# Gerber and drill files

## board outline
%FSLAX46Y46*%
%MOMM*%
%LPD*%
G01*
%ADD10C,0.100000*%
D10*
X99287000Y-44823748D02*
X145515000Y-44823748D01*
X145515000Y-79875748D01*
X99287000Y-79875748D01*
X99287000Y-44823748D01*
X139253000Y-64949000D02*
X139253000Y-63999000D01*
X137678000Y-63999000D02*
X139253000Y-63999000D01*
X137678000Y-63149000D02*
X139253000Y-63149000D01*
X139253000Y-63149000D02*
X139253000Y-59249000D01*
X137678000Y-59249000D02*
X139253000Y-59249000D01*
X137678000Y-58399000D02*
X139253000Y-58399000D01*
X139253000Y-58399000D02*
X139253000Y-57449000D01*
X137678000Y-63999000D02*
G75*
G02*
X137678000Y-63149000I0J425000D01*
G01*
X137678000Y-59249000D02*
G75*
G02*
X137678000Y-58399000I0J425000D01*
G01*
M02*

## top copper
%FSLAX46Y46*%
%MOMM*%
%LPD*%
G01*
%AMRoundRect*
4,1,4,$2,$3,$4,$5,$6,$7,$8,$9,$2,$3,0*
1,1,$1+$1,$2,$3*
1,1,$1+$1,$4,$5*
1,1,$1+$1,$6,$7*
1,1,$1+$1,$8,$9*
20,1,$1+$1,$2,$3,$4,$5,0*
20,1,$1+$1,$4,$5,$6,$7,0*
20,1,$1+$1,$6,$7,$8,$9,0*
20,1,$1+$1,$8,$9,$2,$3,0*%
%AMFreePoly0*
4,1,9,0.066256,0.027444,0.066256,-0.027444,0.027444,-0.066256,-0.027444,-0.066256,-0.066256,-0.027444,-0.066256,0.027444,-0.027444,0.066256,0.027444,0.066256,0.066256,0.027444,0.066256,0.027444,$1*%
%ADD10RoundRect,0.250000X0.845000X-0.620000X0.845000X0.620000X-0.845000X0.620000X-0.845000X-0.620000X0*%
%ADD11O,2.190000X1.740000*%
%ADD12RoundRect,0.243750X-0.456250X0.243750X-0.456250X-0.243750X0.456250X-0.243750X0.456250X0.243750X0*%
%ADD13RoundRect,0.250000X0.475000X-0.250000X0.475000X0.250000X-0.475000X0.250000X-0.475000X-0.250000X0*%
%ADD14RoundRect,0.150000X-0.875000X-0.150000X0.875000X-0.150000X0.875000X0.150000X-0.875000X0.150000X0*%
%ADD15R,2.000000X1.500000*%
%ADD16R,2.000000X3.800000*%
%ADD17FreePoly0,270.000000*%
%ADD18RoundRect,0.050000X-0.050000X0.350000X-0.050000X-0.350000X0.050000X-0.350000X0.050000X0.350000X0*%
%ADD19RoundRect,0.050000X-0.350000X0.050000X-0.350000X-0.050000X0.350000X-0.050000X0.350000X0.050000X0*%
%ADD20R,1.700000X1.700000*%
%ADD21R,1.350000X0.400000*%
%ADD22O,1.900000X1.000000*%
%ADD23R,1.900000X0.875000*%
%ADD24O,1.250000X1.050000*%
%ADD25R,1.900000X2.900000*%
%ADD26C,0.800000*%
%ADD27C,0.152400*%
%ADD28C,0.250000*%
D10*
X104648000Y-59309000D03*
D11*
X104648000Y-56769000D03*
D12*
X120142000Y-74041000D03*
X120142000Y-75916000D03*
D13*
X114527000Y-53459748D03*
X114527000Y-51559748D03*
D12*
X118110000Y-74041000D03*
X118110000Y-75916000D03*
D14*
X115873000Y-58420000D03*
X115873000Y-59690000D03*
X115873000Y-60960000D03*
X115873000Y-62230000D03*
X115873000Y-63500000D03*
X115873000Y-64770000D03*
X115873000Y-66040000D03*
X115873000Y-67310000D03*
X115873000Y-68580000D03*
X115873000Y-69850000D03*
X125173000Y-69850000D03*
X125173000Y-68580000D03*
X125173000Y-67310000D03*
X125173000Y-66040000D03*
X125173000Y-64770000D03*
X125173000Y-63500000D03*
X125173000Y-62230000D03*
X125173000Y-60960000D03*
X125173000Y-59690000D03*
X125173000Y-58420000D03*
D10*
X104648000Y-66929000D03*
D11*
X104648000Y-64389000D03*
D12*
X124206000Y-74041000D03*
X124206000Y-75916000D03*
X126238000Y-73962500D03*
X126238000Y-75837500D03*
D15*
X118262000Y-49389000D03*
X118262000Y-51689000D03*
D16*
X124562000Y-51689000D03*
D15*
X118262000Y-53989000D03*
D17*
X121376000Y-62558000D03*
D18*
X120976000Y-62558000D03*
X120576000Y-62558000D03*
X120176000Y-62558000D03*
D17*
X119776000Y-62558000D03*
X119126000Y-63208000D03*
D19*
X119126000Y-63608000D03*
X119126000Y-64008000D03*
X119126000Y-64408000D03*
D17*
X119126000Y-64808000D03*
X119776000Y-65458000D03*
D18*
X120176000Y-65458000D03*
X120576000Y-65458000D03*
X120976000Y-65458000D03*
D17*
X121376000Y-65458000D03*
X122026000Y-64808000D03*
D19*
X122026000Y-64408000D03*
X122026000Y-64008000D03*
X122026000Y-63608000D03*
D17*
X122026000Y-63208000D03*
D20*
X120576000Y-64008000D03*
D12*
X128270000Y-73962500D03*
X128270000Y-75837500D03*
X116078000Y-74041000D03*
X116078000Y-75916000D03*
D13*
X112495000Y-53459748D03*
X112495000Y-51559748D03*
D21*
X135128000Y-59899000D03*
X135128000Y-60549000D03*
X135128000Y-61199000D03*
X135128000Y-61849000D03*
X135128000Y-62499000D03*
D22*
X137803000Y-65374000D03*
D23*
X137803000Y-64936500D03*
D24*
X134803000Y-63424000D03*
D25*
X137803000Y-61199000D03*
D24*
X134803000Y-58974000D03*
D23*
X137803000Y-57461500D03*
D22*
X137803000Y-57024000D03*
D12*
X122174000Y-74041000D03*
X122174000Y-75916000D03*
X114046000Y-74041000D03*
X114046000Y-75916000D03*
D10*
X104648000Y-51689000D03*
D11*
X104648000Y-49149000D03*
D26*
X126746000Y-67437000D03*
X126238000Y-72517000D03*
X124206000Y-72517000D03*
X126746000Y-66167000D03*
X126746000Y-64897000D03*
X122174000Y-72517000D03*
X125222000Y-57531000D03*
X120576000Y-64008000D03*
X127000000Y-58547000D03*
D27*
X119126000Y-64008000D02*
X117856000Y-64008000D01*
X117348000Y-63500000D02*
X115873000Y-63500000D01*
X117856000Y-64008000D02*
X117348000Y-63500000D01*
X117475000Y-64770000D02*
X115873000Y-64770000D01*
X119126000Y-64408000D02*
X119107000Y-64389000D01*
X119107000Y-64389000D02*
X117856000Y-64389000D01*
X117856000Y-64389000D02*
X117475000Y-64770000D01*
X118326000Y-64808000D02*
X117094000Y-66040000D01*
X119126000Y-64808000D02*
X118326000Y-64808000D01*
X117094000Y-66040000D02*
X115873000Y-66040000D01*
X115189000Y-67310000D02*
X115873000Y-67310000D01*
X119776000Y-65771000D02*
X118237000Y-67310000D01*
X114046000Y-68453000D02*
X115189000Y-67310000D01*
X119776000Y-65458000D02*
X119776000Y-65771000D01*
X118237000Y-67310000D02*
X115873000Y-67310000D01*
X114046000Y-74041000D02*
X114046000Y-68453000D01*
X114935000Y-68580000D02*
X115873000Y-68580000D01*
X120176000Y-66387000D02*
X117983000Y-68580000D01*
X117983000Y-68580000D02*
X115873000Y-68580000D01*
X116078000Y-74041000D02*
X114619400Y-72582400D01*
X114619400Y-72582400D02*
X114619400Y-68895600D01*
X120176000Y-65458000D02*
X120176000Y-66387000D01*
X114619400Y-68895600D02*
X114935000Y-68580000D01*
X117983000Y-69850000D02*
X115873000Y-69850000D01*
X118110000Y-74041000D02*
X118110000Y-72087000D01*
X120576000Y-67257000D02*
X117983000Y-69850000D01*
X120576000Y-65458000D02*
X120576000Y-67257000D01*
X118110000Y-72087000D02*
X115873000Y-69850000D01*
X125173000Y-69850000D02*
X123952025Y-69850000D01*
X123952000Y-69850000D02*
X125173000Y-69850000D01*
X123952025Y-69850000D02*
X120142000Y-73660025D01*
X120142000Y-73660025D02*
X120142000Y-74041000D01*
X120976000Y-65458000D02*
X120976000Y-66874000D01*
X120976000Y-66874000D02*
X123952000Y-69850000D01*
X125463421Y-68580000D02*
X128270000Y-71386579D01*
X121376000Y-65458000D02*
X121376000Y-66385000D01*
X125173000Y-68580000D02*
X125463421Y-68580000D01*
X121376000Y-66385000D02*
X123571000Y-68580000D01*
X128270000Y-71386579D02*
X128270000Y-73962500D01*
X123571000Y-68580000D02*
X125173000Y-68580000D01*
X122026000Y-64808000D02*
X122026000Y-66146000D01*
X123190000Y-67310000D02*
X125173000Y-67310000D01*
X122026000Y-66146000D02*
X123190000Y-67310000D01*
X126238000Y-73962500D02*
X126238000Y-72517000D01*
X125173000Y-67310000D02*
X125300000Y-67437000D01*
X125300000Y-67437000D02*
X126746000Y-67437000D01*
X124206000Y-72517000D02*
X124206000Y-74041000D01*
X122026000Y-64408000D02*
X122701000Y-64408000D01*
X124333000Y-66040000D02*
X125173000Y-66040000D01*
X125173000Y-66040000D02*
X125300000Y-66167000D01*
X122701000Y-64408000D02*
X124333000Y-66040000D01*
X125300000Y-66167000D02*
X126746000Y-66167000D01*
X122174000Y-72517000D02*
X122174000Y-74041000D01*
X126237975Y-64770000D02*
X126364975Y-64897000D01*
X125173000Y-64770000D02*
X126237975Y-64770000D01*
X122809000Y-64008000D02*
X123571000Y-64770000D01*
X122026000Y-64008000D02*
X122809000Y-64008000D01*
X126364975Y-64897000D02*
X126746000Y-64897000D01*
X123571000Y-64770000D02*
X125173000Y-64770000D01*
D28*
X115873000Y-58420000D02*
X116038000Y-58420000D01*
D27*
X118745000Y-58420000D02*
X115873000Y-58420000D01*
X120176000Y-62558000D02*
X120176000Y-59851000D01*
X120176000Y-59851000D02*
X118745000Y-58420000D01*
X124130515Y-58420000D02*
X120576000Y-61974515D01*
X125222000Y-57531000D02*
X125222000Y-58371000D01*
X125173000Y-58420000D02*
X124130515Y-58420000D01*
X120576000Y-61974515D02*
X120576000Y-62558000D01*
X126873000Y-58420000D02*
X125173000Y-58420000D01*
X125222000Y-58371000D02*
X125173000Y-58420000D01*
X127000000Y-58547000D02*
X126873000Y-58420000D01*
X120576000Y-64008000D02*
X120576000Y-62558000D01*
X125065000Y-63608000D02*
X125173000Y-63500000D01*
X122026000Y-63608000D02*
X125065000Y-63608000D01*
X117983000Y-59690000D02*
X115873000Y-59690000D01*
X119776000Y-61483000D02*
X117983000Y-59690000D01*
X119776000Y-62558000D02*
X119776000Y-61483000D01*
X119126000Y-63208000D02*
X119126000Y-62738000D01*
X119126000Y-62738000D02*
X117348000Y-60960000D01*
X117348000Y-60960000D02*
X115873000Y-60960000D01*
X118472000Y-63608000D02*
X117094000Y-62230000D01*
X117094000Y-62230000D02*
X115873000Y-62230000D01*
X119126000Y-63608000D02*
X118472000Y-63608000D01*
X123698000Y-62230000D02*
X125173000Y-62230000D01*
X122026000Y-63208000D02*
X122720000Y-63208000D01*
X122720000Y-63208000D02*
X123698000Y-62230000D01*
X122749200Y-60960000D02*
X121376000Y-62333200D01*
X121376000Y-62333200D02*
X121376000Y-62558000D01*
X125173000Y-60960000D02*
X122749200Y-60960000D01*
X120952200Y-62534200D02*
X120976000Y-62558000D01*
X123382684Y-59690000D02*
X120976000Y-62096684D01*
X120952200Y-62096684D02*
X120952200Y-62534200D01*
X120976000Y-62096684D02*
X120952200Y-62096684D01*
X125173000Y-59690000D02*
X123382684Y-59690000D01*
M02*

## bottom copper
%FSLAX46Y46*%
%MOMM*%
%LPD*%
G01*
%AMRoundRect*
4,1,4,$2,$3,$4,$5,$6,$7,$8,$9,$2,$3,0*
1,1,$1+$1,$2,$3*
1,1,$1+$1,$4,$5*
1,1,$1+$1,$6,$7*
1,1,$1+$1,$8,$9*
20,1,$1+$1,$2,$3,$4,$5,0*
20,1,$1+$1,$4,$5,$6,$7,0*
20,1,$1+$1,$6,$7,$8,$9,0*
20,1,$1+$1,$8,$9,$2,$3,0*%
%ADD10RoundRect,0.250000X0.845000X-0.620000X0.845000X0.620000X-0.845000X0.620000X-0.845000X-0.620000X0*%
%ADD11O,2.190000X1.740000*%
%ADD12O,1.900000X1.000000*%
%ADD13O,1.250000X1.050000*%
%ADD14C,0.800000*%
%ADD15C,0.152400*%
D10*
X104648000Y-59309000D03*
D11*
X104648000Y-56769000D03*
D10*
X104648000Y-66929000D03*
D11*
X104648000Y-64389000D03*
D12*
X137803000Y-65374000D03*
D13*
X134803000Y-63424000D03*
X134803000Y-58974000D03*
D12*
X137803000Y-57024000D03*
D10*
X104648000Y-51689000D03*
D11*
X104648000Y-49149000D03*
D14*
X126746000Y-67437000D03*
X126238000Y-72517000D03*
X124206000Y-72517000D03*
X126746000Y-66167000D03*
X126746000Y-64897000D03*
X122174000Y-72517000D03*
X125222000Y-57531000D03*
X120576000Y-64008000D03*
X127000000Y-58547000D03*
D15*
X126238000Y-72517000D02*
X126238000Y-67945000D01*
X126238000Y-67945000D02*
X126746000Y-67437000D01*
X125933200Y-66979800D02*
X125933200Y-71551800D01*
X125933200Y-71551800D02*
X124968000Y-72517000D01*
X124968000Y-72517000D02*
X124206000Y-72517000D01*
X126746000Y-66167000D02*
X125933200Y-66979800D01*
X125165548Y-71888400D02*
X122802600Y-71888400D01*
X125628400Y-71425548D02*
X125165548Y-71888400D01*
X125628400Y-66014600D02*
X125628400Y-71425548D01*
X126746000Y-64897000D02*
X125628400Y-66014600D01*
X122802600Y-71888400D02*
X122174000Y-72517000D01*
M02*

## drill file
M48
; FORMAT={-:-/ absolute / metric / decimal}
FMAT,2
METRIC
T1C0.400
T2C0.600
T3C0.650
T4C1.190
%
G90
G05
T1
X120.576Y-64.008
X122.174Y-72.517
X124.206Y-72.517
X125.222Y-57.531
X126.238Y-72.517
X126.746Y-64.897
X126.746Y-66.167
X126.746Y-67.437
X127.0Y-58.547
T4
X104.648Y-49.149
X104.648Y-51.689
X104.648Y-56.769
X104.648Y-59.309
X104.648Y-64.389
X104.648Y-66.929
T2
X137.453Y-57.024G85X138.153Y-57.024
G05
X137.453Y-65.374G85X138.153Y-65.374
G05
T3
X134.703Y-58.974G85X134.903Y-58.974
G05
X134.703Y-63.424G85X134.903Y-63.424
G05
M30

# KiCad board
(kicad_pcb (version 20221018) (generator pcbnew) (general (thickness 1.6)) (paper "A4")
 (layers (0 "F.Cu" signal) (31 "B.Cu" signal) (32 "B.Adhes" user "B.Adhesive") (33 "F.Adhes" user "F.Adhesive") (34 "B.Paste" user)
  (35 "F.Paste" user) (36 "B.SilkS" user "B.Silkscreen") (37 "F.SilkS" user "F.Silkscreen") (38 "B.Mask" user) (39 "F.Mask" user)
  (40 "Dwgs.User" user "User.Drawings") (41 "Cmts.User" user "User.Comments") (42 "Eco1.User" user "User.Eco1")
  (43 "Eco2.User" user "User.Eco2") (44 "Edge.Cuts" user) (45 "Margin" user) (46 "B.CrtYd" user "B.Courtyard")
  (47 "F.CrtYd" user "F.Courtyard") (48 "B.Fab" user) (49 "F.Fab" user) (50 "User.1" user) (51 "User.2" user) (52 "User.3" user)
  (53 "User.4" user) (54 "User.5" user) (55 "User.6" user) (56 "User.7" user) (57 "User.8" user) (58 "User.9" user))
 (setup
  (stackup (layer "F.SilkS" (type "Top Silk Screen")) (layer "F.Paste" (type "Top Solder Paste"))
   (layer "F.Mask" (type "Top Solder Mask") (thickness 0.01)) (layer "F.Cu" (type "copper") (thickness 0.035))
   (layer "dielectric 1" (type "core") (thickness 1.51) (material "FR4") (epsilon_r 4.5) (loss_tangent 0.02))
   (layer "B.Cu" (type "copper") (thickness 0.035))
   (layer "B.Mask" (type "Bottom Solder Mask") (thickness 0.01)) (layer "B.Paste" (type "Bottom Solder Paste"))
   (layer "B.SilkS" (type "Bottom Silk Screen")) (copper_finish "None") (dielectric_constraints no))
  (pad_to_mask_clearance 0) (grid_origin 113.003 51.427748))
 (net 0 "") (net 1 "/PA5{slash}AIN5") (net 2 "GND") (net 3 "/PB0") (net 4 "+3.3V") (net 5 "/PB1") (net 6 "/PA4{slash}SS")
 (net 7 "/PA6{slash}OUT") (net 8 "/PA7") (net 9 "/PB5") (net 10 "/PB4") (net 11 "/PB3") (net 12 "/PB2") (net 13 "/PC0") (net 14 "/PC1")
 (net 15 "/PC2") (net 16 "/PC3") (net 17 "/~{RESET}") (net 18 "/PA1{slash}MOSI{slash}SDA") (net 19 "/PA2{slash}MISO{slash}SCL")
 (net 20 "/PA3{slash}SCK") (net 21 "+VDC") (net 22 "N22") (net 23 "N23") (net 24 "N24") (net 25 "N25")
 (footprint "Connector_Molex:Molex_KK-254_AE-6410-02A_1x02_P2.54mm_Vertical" (layer "F.Cu") (at 104.648 59.309 90)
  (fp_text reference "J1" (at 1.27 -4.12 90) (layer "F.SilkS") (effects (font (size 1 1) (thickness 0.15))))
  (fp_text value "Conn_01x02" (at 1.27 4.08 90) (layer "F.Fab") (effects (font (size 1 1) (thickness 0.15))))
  (pad "1" thru_hole roundrect (at 0 0 90) (size 1.74 2.19) (drill 1.19) (layers "*.Cu" "*.Mask") (roundrect_rratio 0.1436781609)
   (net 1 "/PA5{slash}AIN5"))
  (pad "2" thru_hole oval (at 2.54 0 90) (size 1.74 2.19) (drill 1.19) (layers "*.Cu" "*.Mask") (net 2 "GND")))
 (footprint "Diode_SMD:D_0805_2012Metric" (layer "F.Cu") (at 120.142 74.9785 -90)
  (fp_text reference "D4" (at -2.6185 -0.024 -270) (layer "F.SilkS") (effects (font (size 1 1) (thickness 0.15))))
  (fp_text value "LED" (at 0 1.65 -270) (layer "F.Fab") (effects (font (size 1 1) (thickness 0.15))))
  (pad "1" smd roundrect (at -0.9375 0 270) (size 0.975 1.4) (layers "F.Cu" "F.Paste" "F.Mask") (roundrect_rratio 0.25) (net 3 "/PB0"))
  (pad "2" smd roundrect (at 0.9375 0 270) (size 0.975 1.4) (layers "F.Cu" "F.Paste" "F.Mask") (roundrect_rratio 0.25) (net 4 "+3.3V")))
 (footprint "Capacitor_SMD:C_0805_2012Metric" (layer "F.Cu") (at 114.527 52.509748 90)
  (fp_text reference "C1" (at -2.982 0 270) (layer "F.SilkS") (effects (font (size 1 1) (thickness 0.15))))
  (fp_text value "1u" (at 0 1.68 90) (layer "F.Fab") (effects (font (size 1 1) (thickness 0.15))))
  (pad "1" smd roundrect (at -0.95 0 90) (size 1 1.45) (layers "F.Cu" "F.Paste" "F.Mask") (roundrect_rratio 0.25) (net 4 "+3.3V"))
  (pad "2" smd roundrect (at 0.95 0 90) (size 1 1.45) (layers "F.Cu" "F.Paste" "F.Mask") (roundrect_rratio 0.25) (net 2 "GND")))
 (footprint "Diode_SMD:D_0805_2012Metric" (layer "F.Cu") (at 118.11 74.9785 -90)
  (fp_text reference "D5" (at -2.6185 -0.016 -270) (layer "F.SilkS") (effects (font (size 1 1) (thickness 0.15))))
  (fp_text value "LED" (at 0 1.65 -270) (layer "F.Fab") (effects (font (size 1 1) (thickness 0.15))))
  (pad "1" smd roundrect (at -0.9375 0 270) (size 0.975 1.4) (layers "F.Cu" "F.Paste" "F.Mask") (roundrect_rratio 0.25) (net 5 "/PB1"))
  (pad "2" smd roundrect (at 0.9375 0 270) (size 0.975 1.4) (layers "F.Cu" "F.Paste" "F.Mask") (roundrect_rratio 0.25) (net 4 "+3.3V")))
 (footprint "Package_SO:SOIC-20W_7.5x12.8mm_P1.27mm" (layer "F.Cu") (at 120.523 64.135)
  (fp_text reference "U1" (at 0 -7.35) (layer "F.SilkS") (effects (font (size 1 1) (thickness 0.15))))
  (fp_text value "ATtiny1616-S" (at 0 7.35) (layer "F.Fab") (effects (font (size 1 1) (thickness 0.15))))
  (pad "1" smd roundrect (at -4.65 -5.715) (size 2.05 0.6) (layers "F.Cu" "F.Paste" "F.Mask") (roundrect_rratio 0.25) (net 4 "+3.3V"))
  (pad "2" smd roundrect (at -4.65 -4.445) (size 2.05 0.6) (layers "F.Cu" "F.Paste" "F.Mask") (roundrect_rratio 0.25)
   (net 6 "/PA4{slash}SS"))
  (pad "3" smd roundrect (at -4.65 -3.175) (size 2.05 0.6) (layers "F.Cu" "F.Paste" "F.Mask") (roundrect_rratio 0.25)
   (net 1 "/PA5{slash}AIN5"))
  (pad "4" smd roundrect (at -4.65 -1.905) (size 2.05 0.6) (layers "F.Cu" "F.Paste" "F.Mask") (roundrect_rratio 0.25)
   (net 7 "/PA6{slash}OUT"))
  (pad "5" smd roundrect (at -4.65 -0.635) (size 2.05 0.6) (layers "F.Cu" "F.Paste" "F.Mask") (roundrect_rratio 0.25) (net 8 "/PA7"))
  (pad "6" smd roundrect (at -4.65 0.635) (size 2.05 0.6) (layers "F.Cu" "F.Paste" "F.Mask") (roundrect_rratio 0.25) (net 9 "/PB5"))
  (pad "7" smd roundrect (at -4.65 1.905) (size 2.05 0.6) (layers "F.Cu" "F.Paste" "F.Mask") (roundrect_rratio 0.25) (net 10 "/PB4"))
  (pad "8" smd roundrect (at -4.65 3.175) (size 2.05 0.6) (layers "F.Cu" "F.Paste" "F.Mask") (roundrect_rratio 0.25) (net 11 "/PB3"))
  (pad "9" smd roundrect (at -4.65 4.445) (size 2.05 0.6) (layers "F.Cu" "F.Paste" "F.Mask") (roundrect_rratio 0.25) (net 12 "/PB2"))
  (pad "10" smd roundrect (at -4.65 5.715) (size 2.05 0.6) (layers "F.Cu" "F.Paste" "F.Mask") (roundrect_rratio 0.25) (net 5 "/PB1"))
  (pad "11" smd roundrect (at 4.65 5.715) (size 2.05 0.6) (layers "F.Cu" "F.Paste" "F.Mask") (roundrect_rratio 0.25) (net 3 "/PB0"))
  (pad "12" smd roundrect (at 4.65 4.445) (size 2.05 0.6) (layers "F.Cu" "F.Paste" "F.Mask") (roundrect_rratio 0.25) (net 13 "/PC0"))
  (pad "13" smd roundrect (at 4.65 3.175) (size 2.05 0.6) (layers "F.Cu" "F.Paste" "F.Mask") (roundrect_rratio 0.25) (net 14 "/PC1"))
  (pad "14" smd roundrect (at 4.65 1.905) (size 2.05 0.6) (layers "F.Cu" "F.Paste" "F.Mask") (roundrect_rratio 0.25) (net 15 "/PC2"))
  (pad "15" smd roundrect (at 4.65 0.635) (size 2.05 0.6) (layers "F.Cu" "F.Paste" "F.Mask") (roundrect_rratio 0.25) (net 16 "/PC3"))
  (pad "16" smd roundrect (at 4.65 -0.635) (size 2.05 0.6) (layers "F.Cu" "F.Paste" "F.Mask") (roundrect_rratio 0.25) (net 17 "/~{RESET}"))
  (pad "17" smd roundrect (at 4.65 -1.905) (size 2.05 0.6) (layers "F.Cu" "F.Paste" "F.Mask") (roundrect_rratio 0.25)
   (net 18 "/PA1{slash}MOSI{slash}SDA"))
  (pad "18" smd roundrect (at 4.65 -3.175) (size 2.05 0.6) (layers "F.Cu" "F.Paste" "F.Mask") (roundrect_rratio 0.25)
   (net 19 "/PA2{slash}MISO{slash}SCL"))
  (pad "19" smd roundrect (at 4.65 -4.445) (size 2.05 0.6) (layers "F.Cu" "F.Paste" "F.Mask") (roundrect_rratio 0.25)
   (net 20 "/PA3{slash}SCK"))
  (pad "20" smd roundrect (at 4.65 -5.715) (size 2.05 0.6) (layers "F.Cu" "F.Paste" "F.Mask") (roundrect_rratio 0.25) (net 2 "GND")))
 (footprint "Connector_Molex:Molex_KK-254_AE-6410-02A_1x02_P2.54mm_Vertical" (layer "F.Cu") (at 104.648 66.929 90)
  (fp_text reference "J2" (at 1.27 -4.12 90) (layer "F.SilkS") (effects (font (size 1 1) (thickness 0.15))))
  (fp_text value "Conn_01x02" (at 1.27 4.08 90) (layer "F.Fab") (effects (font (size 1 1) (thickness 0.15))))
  (pad "1" thru_hole roundrect (at 0 0 90) (size 1.74 2.19) (drill 1.19) (layers "*.Cu" "*.Mask") (roundrect_rratio 0.1436781609)
   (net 7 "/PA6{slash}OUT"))
  (pad "2" thru_hole oval (at 2.54 0 90) (size 1.74 2.19) (drill 1.19) (layers "*.Cu" "*.Mask") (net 2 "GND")))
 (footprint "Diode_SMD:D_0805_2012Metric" (layer "F.Cu") (at 124.206 74.9785 -90)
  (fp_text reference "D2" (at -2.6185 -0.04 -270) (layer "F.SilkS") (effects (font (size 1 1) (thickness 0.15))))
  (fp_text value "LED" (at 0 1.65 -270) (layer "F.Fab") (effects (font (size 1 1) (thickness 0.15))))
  (pad "1" smd roundrect (at -0.9375 0 270) (size 0.975 1.4) (layers "F.Cu" "F.Paste" "F.Mask") (roundrect_rratio 0.25) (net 15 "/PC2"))
  (pad "2" smd roundrect (at 0.9375 0 270) (size 0.975 1.4) (layers "F.Cu" "F.Paste" "F.Mask") (roundrect_rratio 0.25) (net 4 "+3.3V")))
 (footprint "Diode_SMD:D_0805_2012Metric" (layer "F.Cu") (at 126.238 74.9 -90)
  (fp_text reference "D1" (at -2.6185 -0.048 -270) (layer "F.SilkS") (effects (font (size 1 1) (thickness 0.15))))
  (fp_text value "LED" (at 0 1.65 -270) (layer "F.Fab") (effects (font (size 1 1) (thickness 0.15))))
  (pad "1" smd roundrect (at -0.9375 0 270) (size 0.975 1.4) (layers "F.Cu" "F.Paste" "F.Mask") (roundrect_rratio 0.25) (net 14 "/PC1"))
  (pad "2" smd roundrect (at 0.9375 0 270) (size 0.975 1.4) (layers "F.Cu" "F.Paste" "F.Mask") (roundrect_rratio 0.25) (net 4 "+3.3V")))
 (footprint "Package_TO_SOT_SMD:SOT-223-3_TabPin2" (layer "F.Cu") (at 121.412 51.689)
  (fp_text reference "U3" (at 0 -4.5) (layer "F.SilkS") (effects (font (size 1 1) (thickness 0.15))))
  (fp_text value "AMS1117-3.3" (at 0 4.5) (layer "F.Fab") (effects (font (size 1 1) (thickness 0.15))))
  (pad "1" smd rect (at -3.15 -2.3) (size 2 1.5) (layers "F.Cu" "F.Paste" "F.Mask") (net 2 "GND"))
  (pad "2" smd rect (at -3.15 0) (size 2 1.5) (layers "F.Cu" "F.Paste" "F.Mask") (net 4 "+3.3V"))
  (pad "2" smd rect (at 3.15 0) (size 2 3.8) (layers "F.Cu" "F.Paste" "F.Mask") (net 4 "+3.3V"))
  (pad "3" smd rect (at -3.15 2.3) (size 2 1.5) (layers "F.Cu" "F.Paste" "F.Mask") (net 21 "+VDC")))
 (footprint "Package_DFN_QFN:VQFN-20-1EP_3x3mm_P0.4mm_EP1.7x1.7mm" (layer "F.Cu") (at 120.576 64.008 -90)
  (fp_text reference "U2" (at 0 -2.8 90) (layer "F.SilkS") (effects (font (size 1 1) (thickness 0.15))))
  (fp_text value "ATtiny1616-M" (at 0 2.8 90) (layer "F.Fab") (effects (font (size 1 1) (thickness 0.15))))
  (pad "" smd roundrect (at -0.425 -0.425 270) (size 0.69 0.69) (layers "F.Paste") (roundrect_rratio 0.25))
  (pad "" smd roundrect (at -0.425 0.425 270) (size 0.69 0.69) (layers "F.Paste") (roundrect_rratio 0.25))
  (pad "" smd roundrect (at 0.425 -0.425 270) (size 0.69 0.69) (layers "F.Paste") (roundrect_rratio 0.25))
  (pad "" smd roundrect (at 0.425 0.425 270) (size 0.69 0.69) (layers "F.Paste") (roundrect_rratio 0.25))
  (pad "1" smd custom (at -1.45 -0.8 270) (size 0.143431 0.143431) (layers "F.Cu" "F.Paste" "F.Mask") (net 19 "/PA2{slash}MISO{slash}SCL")
   (thermal_bridge_angle 45) (options (clearance outline) (anchor circle)) (primitives))
  (pad "2" smd roundrect (at -1.45 -0.4 270) (size 0.8 0.2) (layers "F.Cu" "F.Paste" "F.Mask") (roundrect_rratio 0.25)
   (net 20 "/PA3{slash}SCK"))
  (pad "3" smd roundrect (at -1.45 0 270) (size 0.8 0.2) (layers "F.Cu" "F.Paste" "F.Mask") (roundrect_rratio 0.25) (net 2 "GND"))
  (pad "4" smd roundrect (at -1.45 0.4 270) (size 0.8 0.2) (layers "F.Cu" "F.Paste" "F.Mask") (roundrect_rratio 0.25) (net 4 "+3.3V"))
  (pad "5" smd custom (at -1.45 0.8 270) (size 0.143431 0.143431) (layers "F.Cu" "F.Paste" "F.Mask") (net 6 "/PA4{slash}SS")
   (thermal_bridge_angle 45) (options (clearance outline) (anchor circle)) (primitives))
  (pad "6" smd custom (at -0.8 1.45 270) (size 0.143431 0.143431) (layers "F.Cu" "F.Paste" "F.Mask") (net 1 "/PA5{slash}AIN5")
   (thermal_bridge_angle 45) (options (clearance outline) (anchor circle)) (primitives))
  (pad "7" smd roundrect (at -0.4 1.45 270) (size 0.2 0.8) (layers "F.Cu" "F.Paste" "F.Mask") (roundrect_rratio 0.25)
   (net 7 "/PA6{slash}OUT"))
  (pad "8" smd roundrect (at 0 1.45 270) (size 0.2 0.8) (layers "F.Cu" "F.Paste" "F.Mask") (roundrect_rratio 0.25) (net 8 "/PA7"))
  (pad "9" smd roundrect (at 0.4 1.45 270) (size 0.2 0.8) (layers "F.Cu" "F.Paste" "F.Mask") (roundrect_rratio 0.25) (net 9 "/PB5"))
  (pad "10" smd custom (at 0.8 1.45 270) (size 0.143431 0.143431) (layers "F.Cu" "F.Paste" "F.Mask") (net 10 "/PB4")
   (thermal_bridge_angle 45) (options (clearance outline) (anchor circle)) (primitives))
  (pad "11" smd custom (at 1.45 0.8 270) (size 0.143431 0.143431) (layers "F.Cu" "F.Paste" "F.Mask") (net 11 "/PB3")
   (thermal_bridge_angle 45) (options (clearance outline) (anchor circle)) (primitives))
  (pad "12" smd roundrect (at 1.45 0.4 270) (size 0.8 0.2) (layers "F.Cu" "F.Paste" "F.Mask") (roundrect_rratio 0.25) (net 12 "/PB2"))
  (pad "13" smd roundrect (at 1.45 0 270) (size 0.8 0.2) (layers "F.Cu" "F.Paste" "F.Mask") (roundrect_rratio 0.25) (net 5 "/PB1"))
  (pad "14" smd roundrect (at 1.45 -0.4 270) (size 0.8 0.2) (layers "F.Cu" "F.Paste" "F.Mask") (roundrect_rratio 0.25) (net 3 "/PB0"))
  (pad "15" smd custom (at 1.45 -0.8 270) (size 0.143431 0.143431) (layers "F.Cu" "F.Paste" "F.Mask") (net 13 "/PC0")
   (thermal_bridge_angle 45) (options (clearance outline) (anchor circle)) (primitives))
  (pad "16" smd custom (at 0.8 -1.45 270) (size 0.143431 0.143431) (layers "F.Cu" "F.Paste" "F.Mask") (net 14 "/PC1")
   (thermal_bridge_angle 45) (options (clearance outline) (anchor circle)) (primitives))
  (pad "17" smd roundrect (at 0.4 -1.45 270) (size 0.2 0.8) (layers "F.Cu" "F.Paste" "F.Mask") (roundrect_rratio 0.25) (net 15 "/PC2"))
  (pad "18" smd roundrect (at 0 -1.45 270) (size 0.2 0.8) (layers "F.Cu" "F.Paste" "F.Mask") (roundrect_rratio 0.25) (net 16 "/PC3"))
  (pad "19" smd roundrect (at -0.4 -1.45 270) (size 0.2 0.8) (layers "F.Cu" "F.Paste" "F.Mask") (roundrect_rratio 0.25) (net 17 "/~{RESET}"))
  (pad "20" smd custom (at -0.8 -1.45 270) (size 0.143431 0.143431) (layers "F.Cu" "F.Paste" "F.Mask") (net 18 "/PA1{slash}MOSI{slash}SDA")
   (thermal_bridge_angle 45) (options (clearance outline) (anchor circle)) (primitives))
  (pad "21" smd rect (at 0 0 270) (size 1.7 1.7) (layers "F.Cu" "F.Mask") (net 2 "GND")))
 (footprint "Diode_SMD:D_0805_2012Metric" (layer "F.Cu") (at 128.27 74.9 -90)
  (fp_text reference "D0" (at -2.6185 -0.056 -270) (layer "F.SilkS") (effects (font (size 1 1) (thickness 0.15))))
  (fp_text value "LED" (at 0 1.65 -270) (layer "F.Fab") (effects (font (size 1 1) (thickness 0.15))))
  (pad "1" smd roundrect (at -0.9375 0 270) (size 0.975 1.4) (layers "F.Cu" "F.Paste" "F.Mask") (roundrect_rratio 0.25) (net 13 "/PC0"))
  (pad "2" smd roundrect (at 0.9375 0 270) (size 0.975 1.4) (layers "F.Cu" "F.Paste" "F.Mask") (roundrect_rratio 0.25) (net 4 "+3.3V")))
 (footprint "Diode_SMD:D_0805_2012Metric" (layer "F.Cu") (at 116.078 74.9785 -90)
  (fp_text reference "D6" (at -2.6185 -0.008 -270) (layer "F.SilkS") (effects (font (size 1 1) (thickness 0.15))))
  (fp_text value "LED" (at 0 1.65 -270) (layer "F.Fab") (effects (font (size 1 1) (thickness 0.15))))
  (pad "1" smd roundrect (at -0.9375 0 270) (size 0.975 1.4) (layers "F.Cu" "F.Paste" "F.Mask") (roundrect_rratio 0.25) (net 12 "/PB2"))
  (pad "2" smd roundrect (at 0.9375 0 270) (size 0.975 1.4) (layers "F.Cu" "F.Paste" "F.Mask") (roundrect_rratio 0.25) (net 4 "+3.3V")))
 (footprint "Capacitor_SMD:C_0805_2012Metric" (layer "F.Cu") (at 112.495 52.509748 90)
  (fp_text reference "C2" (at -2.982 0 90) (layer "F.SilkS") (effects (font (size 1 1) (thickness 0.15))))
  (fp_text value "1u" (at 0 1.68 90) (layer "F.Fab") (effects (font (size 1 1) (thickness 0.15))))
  (pad "1" smd roundrect (at -0.95 0 90) (size 1 1.45) (layers "F.Cu" "F.Paste" "F.Mask") (roundrect_rratio 0.25) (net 21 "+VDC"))
  (pad "2" smd roundrect (at 0.95 0 90) (size 1 1.45) (layers "F.Cu" "F.Paste" "F.Mask") (roundrect_rratio 0.25) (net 2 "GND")))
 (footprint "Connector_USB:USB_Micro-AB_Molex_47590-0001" (layer "F.Cu") (at 137.803 61.199 90)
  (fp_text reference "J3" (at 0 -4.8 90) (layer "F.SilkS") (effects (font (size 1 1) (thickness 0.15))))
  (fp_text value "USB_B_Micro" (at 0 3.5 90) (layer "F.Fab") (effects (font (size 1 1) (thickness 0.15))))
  (fp_line (start -3.75 1.45) (end -2.8 1.45) (stroke (width 0.1) (type solid)) (layer "Edge.Cuts"))
  (fp_line (start -2.8 -0.125) (end -2.8 1.45) (stroke (width 0.1) (type solid)) (layer "Edge.Cuts"))
  (fp_line (start -1.95 -0.125) (end -1.95 1.45) (stroke (width 0.1) (type solid)) (layer "Edge.Cuts"))
  (fp_line (start -1.95 1.45) (end 1.95 1.45) (stroke (width 0.1) (type solid)) (layer "Edge.Cuts"))
  (fp_line (start 1.95 -0.125) (end 1.95 1.45) (stroke (width 0.1) (type solid)) (layer "Edge.Cuts"))
  (fp_line (start 2.8 -0.125) (end 2.8 1.45) (stroke (width 0.1) (type solid)) (layer "Edge.Cuts"))
  (fp_line (start 2.8 1.45) (end 3.75 1.45) (stroke (width 0.1) (type solid)) (layer "Edge.Cuts"))
  (fp_arc (start -2.8 -0.125) (mid -2.375 -0.55) (end -1.95 -0.125) (stroke (width 0.1) (type solid)) (layer "Edge.Cuts"))
  (fp_arc (start 1.95 -0.125) (mid 2.375 -0.55) (end 2.8 -0.125) (stroke (width 0.1) (type solid)) (layer "Edge.Cuts"))
  (pad "" smd rect (at -3.5 0 90) (size 0.3 0.85) (layers "F.Paste"))
  (pad "" smd rect (at 3.5 0 90) (size 0.3 0.85) (layers "F.Paste"))
  (pad "1" smd rect (at 1.3 -2.675 90) (size 0.4 1.35) (layers "F.Cu" "F.Paste" "F.Mask") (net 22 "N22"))
  (pad "2" smd rect (at 0.65 -2.675 90) (size 0.4 1.35) (layers "F.Cu" "F.Paste" "F.Mask") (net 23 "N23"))
  (pad "3" smd rect (at 0 -2.675 90) (size 0.4 1.35) (layers "F.Cu" "F.Paste" "F.Mask") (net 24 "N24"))
  (pad "4" smd rect (at -0.65 -2.675 90) (size 0.4 1.35) (layers "F.Cu" "F.Paste" "F.Mask") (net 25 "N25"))
  (pad "5" smd rect (at -1.3 -2.675 90) (size 0.4 1.35) (layers "F.Cu" "F.Paste" "F.Mask") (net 2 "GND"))
  (pad "6" thru_hole oval (at -4.175 0 90) (size 1 1.9) (drill oval 0.6 1.3) (layers "*.Cu" "*.Mask") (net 2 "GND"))
  (pad "6" smd rect (at -3.7375 0 90) (size 0.875 1.9) (layers "F.Cu" "F.Mask") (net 2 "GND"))
  (pad "6" thru_hole oval (at -2.225 -3 90) (size 1.05 1.25) (drill oval 0.65 0.85) (layers "*.Cu" "*.Mask") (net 2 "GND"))
  (pad "6" smd rect (at 0 0 90) (size 2.9 1.9) (layers "F.Cu" "F.Paste" "F.Mask") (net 2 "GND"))
  (pad "6" thru_hole oval (at 2.225 -3 90) (size 1.05 1.25) (drill oval 0.65 0.85) (layers "*.Cu" "*.Mask") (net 2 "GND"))
  (pad "6" smd rect (at 3.7375 0 90) (size 0.875 1.9) (layers "F.Cu" "F.Mask") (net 2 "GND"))
  (pad "6" thru_hole oval (at 4.175 0 90) (size 1 1.9) (drill oval 0.6 1.3) (layers "*.Cu" "*.Mask") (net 2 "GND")))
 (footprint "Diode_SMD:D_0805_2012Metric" (layer "F.Cu") (at 122.174 74.9785 -90)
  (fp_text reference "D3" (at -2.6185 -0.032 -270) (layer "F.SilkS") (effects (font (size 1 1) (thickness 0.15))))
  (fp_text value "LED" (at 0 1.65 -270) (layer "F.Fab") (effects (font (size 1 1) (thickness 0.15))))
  (pad "1" smd roundrect (at -0.9375 0 270) (size 0.975 1.4) (layers "F.Cu" "F.Paste" "F.Mask") (roundrect_rratio 0.25) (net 16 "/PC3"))
  (pad "2" smd roundrect (at 0.9375 0 270) (size 0.975 1.4) (layers "F.Cu" "F.Paste" "F.Mask") (roundrect_rratio 0.25) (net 4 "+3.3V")))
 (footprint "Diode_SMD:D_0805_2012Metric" (layer "F.Cu") (at 114.046 74.9785 -90)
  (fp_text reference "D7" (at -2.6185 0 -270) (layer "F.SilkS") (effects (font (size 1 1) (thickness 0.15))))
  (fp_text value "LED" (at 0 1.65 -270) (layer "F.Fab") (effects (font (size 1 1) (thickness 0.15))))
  (pad "1" smd roundrect (at -0.9375 0 270) (size 0.975 1.4) (layers "F.Cu" "F.Paste" "F.Mask") (roundrect_rratio 0.25) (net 11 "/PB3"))
  (pad "2" smd roundrect (at 0.9375 0 270) (size 0.975 1.4) (layers "F.Cu" "F.Paste" "F.Mask") (roundrect_rratio 0.25) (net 4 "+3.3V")))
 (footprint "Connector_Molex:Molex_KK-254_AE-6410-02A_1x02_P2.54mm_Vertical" (layer "F.Cu") (at 104.648 51.689 90)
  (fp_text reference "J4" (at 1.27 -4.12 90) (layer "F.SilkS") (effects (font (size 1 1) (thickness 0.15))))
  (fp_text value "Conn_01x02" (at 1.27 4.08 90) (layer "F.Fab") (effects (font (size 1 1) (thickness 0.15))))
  (pad "1" thru_hole roundrect (at 0 0 90) (size 1.74 2.19) (drill 1.19) (layers "*.Cu" "*.Mask") (roundrect_rratio 0.1436781609)
   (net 21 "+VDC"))
  (pad "2" thru_hole oval (at 2.54 0 90) (size 1.74 2.19) (drill 1.19) (layers "*.Cu" "*.Mask") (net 2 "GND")))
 (gr_rect (start 99.287 44.823748) (end 145.515 79.875748) (stroke (width 0.1) (type default)) (fill none) (layer "Edge.Cuts"))
 (segment (start 119.126 64.008) (end 117.856 64.008) (width 0.1524) (layer "F.Cu") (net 8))
 (segment (start 117.348 63.5) (end 115.873 63.5) (width 0.1524) (layer "F.Cu") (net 8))
 (segment (start 117.856 64.008) (end 117.348 63.5) (width 0.1524) (layer "F.Cu") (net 8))
 (segment (start 117.475 64.77) (end 115.873 64.77) (width 0.1524) (layer "F.Cu") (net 9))
 (segment (start 119.126 64.408) (end 119.107 64.389) (width 0.1524) (layer "F.Cu") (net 9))
 (segment (start 119.107 64.389) (end 117.856 64.389) (width 0.1524) (layer "F.Cu") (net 9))
 (segment (start 117.856 64.389) (end 117.475 64.77) (width 0.1524) (layer "F.Cu") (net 9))
 (segment (start 118.326 64.808) (end 117.094 66.04) (width 0.1524) (layer "F.Cu") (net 10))
 (segment (start 119.126 64.808) (end 118.326 64.808) (width 0.1524) (layer "F.Cu") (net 10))
 (segment (start 117.094 66.04) (end 115.873 66.04) (width 0.1524) (layer "F.Cu") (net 10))
 (segment (start 115.189 67.31) (end 115.873 67.31) (width 0.1524) (layer "F.Cu") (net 11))
 (segment (start 119.776 65.771) (end 118.237 67.31) (width 0.1524) (layer "F.Cu") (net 11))
 (segment (start 114.046 68.453) (end 115.189 67.31) (width 0.1524) (layer "F.Cu") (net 11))
 (segment (start 119.776 65.458) (end 119.776 65.771) (width 0.1524) (layer "F.Cu") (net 11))
 (segment (start 118.237 67.31) (end 115.873 67.31) (width 0.1524) (layer "F.Cu") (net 11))
 (segment (start 114.046 74.041) (end 114.046 68.453) (width 0.1524) (layer "F.Cu") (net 11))
 (segment (start 114.935 68.58) (end 115.873 68.58) (width 0.1524) (layer "F.Cu") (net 12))
 (segment (start 120.176 66.387) (end 117.983 68.58) (width 0.1524) (layer "F.Cu") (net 12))
 (segment (start 117.983 68.58) (end 115.873 68.58) (width 0.1524) (layer "F.Cu") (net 12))
 (segment (start 116.078 74.041) (end 114.6194 72.5824) (width 0.1524) (layer "F.Cu") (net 12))
 (segment (start 114.6194 72.5824) (end 114.6194 68.8956) (width 0.1524) (layer "F.Cu") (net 12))
 (segment (start 120.176 65.458) (end 120.176 66.387) (width 0.1524) (layer "F.Cu") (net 12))
 (segment (start 114.6194 68.8956) (end 114.935 68.58) (width 0.1524) (layer "F.Cu") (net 12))
 (segment (start 117.983 69.85) (end 115.873 69.85) (width 0.1524) (layer "F.Cu") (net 5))
 (segment (start 118.11 74.041) (end 118.11 72.087) (width 0.1524) (layer "F.Cu") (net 5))
 (segment (start 120.576 67.257) (end 117.983 69.85) (width 0.1524) (layer "F.Cu") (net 5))
 (segment (start 120.576 65.458) (end 120.576 67.257) (width 0.1524) (layer "F.Cu") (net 5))
 (segment (start 118.11 72.087) (end 115.873 69.85) (width 0.1524) (layer "F.Cu") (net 5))
 (segment (start 125.173 69.85) (end 123.952025 69.85) (width 0.1524) (layer "F.Cu") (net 3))
 (segment (start 123.952 69.85) (end 125.173 69.85) (width 0.1524) (layer "F.Cu") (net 3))
 (segment (start 123.952025 69.85) (end 120.142 73.660025) (width 0.1524) (layer "F.Cu") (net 3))
 (segment (start 120.142 73.660025) (end 120.142 74.041) (width 0.1524) (layer "F.Cu") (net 3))
 (segment (start 120.976 65.458) (end 120.976 66.874) (width 0.1524) (layer "F.Cu") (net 3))
 (segment (start 120.976 66.874) (end 123.952 69.85) (width 0.1524) (layer "F.Cu") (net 3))
 (segment (start 125.463421 68.58) (end 128.27 71.386579) (width 0.1524) (layer "F.Cu") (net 13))
 (segment (start 121.376 65.458) (end 121.376 66.385) (width 0.1524) (layer "F.Cu") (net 13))
 (segment (start 125.173 68.58) (end 125.463421 68.58) (width 0.1524) (layer "F.Cu") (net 13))
 (segment (start 121.376 66.385) (end 123.571 68.58) (width 0.1524) (layer "F.Cu") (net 13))
 (segment (start 128.27 71.386579) (end 128.27 73.9625) (width 0.1524) (layer "F.Cu") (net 13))
 (segment (start 123.571 68.58) (end 125.173 68.58) (width 0.1524) (layer "F.Cu") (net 13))
 (segment (start 122.026 64.808) (end 122.026 66.146) (width 0.1524) (layer "F.Cu") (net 14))
 (segment (start 123.19 67.31) (end 125.173 67.31) (width 0.1524) (layer "F.Cu") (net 14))
 (segment (start 122.026 66.146) (end 123.19 67.31) (width 0.1524) (layer "F.Cu") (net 14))
 (segment (start 126.238 73.9625) (end 126.238 72.517) (width 0.1524) (layer "F.Cu") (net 14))
 (segment (start 125.173 67.31) (end 125.3 67.437) (width 0.1524) (layer "F.Cu") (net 14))
 (segment (start 125.3 67.437) (end 126.746 67.437) (width 0.1524) (layer "F.Cu") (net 14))
 (via (at 126.746 67.437) (size 0.8) (drill 0.4) (layers "F.Cu" "B.Cu") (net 14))
 (via (at 126.238 72.517) (size 0.8) (drill 0.4) (layers "F.Cu" "B.Cu") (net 14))
 (segment (start 126.238 72.517) (end 126.238 67.945) (width 0.1524) (layer "B.Cu") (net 14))
 (segment (start 126.238 67.945) (end 126.746 67.437) (width 0.1524) (layer "B.Cu") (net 14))
 (segment (start 124.206 72.517) (end 124.206 74.041) (width 0.1524) (layer "F.Cu") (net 15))
 (segment (start 122.026 64.408) (end 122.701 64.408) (width 0.1524) (layer "F.Cu") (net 15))
 (segment (start 124.333 66.04) (end 125.173 66.04) (width 0.1524) (layer "F.Cu") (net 15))
 (segment (start 125.173 66.04) (end 125.3 66.167) (width 0.1524) (layer "F.Cu") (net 15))
 (segment (start 122.701 64.408) (end 124.333 66.04) (width 0.1524) (layer "F.Cu") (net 15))
 (segment (start 125.3 66.167) (end 126.746 66.167) (width 0.1524) (layer "F.Cu") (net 15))
 (via (at 124.206 72.517) (size 0.8) (drill 0.4) (layers "F.Cu" "B.Cu") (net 15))
 (via (at 126.746 66.167) (size 0.8) (drill 0.4) (layers "F.Cu" "B.Cu") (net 15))
 (segment (start 125.9332 66.9798) (end 125.9332 71.5518) (width 0.1524) (layer "B.Cu") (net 15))
 (segment (start 125.9332 71.5518) (end 124.968 72.517) (width 0.1524) (layer "B.Cu") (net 15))
 (segment (start 124.968 72.517) (end 124.206 72.517) (width 0.1524) (layer "B.Cu") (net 15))
 (segment (start 126.746 66.167) (end 125.9332 66.9798) (width 0.1524) (layer "B.Cu") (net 15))
 (segment (start 122.174 72.517) (end 122.174 74.041) (width 0.1524) (layer "F.Cu") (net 16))
 (segment (start 126.237975 64.77) (end 126.364975 64.897) (width 0.1524) (layer "F.Cu") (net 16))
 (segment (start 125.173 64.77) (end 126.237975 64.77) (width 0.1524) (layer "F.Cu") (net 16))
 (segment (start 122.809 64.008) (end 123.571 64.77) (width 0.1524) (layer "F.Cu") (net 16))
 (segment (start 122.026 64.008) (end 122.809 64.008) (width 0.1524) (layer "F.Cu") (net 16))
 (segment (start 126.364975 64.897) (end 126.746 64.897) (width 0.1524) (layer "F.Cu") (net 16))
 (segment (start 123.571 64.77) (end 125.173 64.77) (width 0.1524) (layer "F.Cu") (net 16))
 (via (at 126.746 64.897) (size 0.8) (drill 0.4) (layers "F.Cu" "B.Cu") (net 16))
 (via (at 122.174 72.517) (size 0.8) (drill 0.4) (layers "F.Cu" "B.Cu") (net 16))
 (segment (start 125.165548 71.8884) (end 122.8026 71.8884) (width 0.1524) (layer "B.Cu") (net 16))
 (segment (start 125.6284 71.425548) (end 125.165548 71.8884) (width 0.1524) (layer "B.Cu") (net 16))
 (segment (start 125.6284 66.0146) (end 125.6284 71.425548) (width 0.1524) (layer "B.Cu") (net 16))
 (segment (start 126.746 64.897) (end 125.6284 66.0146) (width 0.1524) (layer "B.Cu") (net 16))
 (segment (start 122.8026 71.8884) (end 122.174 72.517) (width 0.1524) (layer "B.Cu") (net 16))
 (segment (start 115.873 58.42) (end 116.038 58.42) (width 0.25) (layer "F.Cu") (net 4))
 (segment (start 118.745 58.42) (end 115.873 58.42) (width 0.1524) (layer "F.Cu") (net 4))
 (segment (start 120.176 62.558) (end 120.176 59.851) (width 0.1524) (layer "F.Cu") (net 4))
 (segment (start 120.176 59.851) (end 118.745 58.42) (width 0.1524) (layer "F.Cu") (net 4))
 (segment (start 124.130515 58.42) (end 120.576 61.974515) (width 0.1524) (layer "F.Cu") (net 2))
 (segment (start 125.222 57.531) (end 125.222 58.371) (width 0.1524) (layer "F.Cu") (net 2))
 (segment (start 125.173 58.42) (end 124.130515 58.42) (width 0.1524) (layer "F.Cu") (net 2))
 (segment (start 120.576 61.974515) (end 120.576 62.558) (width 0.1524) (layer "F.Cu") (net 2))
 (segment (start 126.873 58.42) (end 125.173 58.42) (width 0.1524) (layer "F.Cu") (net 2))
 (segment (start 125.222 58.371) (end 125.173 58.42) (width 0.1524) (layer "F.Cu") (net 2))
 (segment (start 127 58.547) (end 126.873 58.42) (width 0.1524) (layer "F.Cu") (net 2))
 (segment (start 120.576 64.008) (end 120.576 62.558) (width 0.1524) (layer "F.Cu") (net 2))
 (via (at 125.222 57.531) (size 0.8) (drill 0.4) (layers "F.Cu" "B.Cu") (free) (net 2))
 (via (at 120.576 64.008) (size 0.8) (drill 0.4) (layers "F.Cu" "B.Cu") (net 2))
 (via (at 127 58.547) (size 0.8) (drill 0.4) (layers "F.Cu" "B.Cu") (free) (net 2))
 (segment (start 125.065 63.608) (end 125.173 63.5) (width 0.1524) (layer "F.Cu") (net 17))
 (segment (start 122.026 63.608) (end 125.065 63.608) (width 0.1524) (layer "F.Cu") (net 17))
 (segment (start 117.983 59.69) (end 115.873 59.69) (width 0.1524) (layer "F.Cu") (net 6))
 (segment (start 119.776 61.483) (end 117.983 59.69) (width 0.1524) (layer "F.Cu") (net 6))
 (segment (start 119.776 62.558) (end 119.776 61.483) (width 0.1524) (layer "F.Cu") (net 6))
 (segment (start 119.126 63.208) (end 119.126 62.738) (width 0.1524) (layer "F.Cu") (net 1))
 (segment (start 119.126 62.738) (end 117.348 60.96) (width 0.1524) (layer "F.Cu") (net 1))
 (segment (start 117.348 60.96) (end 115.873 60.96) (width 0.1524) (layer "F.Cu") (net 1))
 (segment (start 118.472 63.608) (end 117.094 62.23) (width 0.1524) (layer "F.Cu") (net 7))
 (segment (start 117.094 62.23) (end 115.873 62.23) (width 0.1524) (layer "F.Cu") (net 7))
 (segment (start 119.126 63.608) (end 118.472 63.608) (width 0.1524) (layer "F.Cu") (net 7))
 (segment (start 123.698 62.23) (end 125.173 62.23) (width 0.1524) (layer "F.Cu") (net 18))
 (segment (start 122.026 63.208) (end 122.72 63.208) (width 0.1524) (layer "F.Cu") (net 18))
 (segment (start 122.72 63.208) (end 123.698 62.23) (width 0.1524) (layer "F.Cu") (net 18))
 (segment (start 122.7492 60.96) (end 121.376 62.3332) (width 0.1524) (layer "F.Cu") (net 19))
 (segment (start 121.376 62.3332) (end 121.376 62.558) (width 0.1524) (layer "F.Cu") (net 19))
 (segment (start 125.173 60.96) (end 122.7492 60.96) (width 0.1524) (layer "F.Cu") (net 19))
 (segment (start 120.9522 62.5342) (end 120.976 62.558) (width 0.1524) (layer "F.Cu") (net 20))
 (segment (start 123.382684 59.69) (end 120.976 62.096684) (width 0.1524) (layer "F.Cu") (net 20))
 (segment (start 120.9522 62.096684) (end 120.9522 62.5342) (width 0.1524) (layer "F.Cu") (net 20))
 (segment (start 120.976 62.096684) (end 120.9522 62.096684) (width 0.1524) (layer "F.Cu") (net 20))
 (segment (start 125.173 59.69) (end 123.382684 59.69) (width 0.1524) (layer "F.Cu") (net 20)))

